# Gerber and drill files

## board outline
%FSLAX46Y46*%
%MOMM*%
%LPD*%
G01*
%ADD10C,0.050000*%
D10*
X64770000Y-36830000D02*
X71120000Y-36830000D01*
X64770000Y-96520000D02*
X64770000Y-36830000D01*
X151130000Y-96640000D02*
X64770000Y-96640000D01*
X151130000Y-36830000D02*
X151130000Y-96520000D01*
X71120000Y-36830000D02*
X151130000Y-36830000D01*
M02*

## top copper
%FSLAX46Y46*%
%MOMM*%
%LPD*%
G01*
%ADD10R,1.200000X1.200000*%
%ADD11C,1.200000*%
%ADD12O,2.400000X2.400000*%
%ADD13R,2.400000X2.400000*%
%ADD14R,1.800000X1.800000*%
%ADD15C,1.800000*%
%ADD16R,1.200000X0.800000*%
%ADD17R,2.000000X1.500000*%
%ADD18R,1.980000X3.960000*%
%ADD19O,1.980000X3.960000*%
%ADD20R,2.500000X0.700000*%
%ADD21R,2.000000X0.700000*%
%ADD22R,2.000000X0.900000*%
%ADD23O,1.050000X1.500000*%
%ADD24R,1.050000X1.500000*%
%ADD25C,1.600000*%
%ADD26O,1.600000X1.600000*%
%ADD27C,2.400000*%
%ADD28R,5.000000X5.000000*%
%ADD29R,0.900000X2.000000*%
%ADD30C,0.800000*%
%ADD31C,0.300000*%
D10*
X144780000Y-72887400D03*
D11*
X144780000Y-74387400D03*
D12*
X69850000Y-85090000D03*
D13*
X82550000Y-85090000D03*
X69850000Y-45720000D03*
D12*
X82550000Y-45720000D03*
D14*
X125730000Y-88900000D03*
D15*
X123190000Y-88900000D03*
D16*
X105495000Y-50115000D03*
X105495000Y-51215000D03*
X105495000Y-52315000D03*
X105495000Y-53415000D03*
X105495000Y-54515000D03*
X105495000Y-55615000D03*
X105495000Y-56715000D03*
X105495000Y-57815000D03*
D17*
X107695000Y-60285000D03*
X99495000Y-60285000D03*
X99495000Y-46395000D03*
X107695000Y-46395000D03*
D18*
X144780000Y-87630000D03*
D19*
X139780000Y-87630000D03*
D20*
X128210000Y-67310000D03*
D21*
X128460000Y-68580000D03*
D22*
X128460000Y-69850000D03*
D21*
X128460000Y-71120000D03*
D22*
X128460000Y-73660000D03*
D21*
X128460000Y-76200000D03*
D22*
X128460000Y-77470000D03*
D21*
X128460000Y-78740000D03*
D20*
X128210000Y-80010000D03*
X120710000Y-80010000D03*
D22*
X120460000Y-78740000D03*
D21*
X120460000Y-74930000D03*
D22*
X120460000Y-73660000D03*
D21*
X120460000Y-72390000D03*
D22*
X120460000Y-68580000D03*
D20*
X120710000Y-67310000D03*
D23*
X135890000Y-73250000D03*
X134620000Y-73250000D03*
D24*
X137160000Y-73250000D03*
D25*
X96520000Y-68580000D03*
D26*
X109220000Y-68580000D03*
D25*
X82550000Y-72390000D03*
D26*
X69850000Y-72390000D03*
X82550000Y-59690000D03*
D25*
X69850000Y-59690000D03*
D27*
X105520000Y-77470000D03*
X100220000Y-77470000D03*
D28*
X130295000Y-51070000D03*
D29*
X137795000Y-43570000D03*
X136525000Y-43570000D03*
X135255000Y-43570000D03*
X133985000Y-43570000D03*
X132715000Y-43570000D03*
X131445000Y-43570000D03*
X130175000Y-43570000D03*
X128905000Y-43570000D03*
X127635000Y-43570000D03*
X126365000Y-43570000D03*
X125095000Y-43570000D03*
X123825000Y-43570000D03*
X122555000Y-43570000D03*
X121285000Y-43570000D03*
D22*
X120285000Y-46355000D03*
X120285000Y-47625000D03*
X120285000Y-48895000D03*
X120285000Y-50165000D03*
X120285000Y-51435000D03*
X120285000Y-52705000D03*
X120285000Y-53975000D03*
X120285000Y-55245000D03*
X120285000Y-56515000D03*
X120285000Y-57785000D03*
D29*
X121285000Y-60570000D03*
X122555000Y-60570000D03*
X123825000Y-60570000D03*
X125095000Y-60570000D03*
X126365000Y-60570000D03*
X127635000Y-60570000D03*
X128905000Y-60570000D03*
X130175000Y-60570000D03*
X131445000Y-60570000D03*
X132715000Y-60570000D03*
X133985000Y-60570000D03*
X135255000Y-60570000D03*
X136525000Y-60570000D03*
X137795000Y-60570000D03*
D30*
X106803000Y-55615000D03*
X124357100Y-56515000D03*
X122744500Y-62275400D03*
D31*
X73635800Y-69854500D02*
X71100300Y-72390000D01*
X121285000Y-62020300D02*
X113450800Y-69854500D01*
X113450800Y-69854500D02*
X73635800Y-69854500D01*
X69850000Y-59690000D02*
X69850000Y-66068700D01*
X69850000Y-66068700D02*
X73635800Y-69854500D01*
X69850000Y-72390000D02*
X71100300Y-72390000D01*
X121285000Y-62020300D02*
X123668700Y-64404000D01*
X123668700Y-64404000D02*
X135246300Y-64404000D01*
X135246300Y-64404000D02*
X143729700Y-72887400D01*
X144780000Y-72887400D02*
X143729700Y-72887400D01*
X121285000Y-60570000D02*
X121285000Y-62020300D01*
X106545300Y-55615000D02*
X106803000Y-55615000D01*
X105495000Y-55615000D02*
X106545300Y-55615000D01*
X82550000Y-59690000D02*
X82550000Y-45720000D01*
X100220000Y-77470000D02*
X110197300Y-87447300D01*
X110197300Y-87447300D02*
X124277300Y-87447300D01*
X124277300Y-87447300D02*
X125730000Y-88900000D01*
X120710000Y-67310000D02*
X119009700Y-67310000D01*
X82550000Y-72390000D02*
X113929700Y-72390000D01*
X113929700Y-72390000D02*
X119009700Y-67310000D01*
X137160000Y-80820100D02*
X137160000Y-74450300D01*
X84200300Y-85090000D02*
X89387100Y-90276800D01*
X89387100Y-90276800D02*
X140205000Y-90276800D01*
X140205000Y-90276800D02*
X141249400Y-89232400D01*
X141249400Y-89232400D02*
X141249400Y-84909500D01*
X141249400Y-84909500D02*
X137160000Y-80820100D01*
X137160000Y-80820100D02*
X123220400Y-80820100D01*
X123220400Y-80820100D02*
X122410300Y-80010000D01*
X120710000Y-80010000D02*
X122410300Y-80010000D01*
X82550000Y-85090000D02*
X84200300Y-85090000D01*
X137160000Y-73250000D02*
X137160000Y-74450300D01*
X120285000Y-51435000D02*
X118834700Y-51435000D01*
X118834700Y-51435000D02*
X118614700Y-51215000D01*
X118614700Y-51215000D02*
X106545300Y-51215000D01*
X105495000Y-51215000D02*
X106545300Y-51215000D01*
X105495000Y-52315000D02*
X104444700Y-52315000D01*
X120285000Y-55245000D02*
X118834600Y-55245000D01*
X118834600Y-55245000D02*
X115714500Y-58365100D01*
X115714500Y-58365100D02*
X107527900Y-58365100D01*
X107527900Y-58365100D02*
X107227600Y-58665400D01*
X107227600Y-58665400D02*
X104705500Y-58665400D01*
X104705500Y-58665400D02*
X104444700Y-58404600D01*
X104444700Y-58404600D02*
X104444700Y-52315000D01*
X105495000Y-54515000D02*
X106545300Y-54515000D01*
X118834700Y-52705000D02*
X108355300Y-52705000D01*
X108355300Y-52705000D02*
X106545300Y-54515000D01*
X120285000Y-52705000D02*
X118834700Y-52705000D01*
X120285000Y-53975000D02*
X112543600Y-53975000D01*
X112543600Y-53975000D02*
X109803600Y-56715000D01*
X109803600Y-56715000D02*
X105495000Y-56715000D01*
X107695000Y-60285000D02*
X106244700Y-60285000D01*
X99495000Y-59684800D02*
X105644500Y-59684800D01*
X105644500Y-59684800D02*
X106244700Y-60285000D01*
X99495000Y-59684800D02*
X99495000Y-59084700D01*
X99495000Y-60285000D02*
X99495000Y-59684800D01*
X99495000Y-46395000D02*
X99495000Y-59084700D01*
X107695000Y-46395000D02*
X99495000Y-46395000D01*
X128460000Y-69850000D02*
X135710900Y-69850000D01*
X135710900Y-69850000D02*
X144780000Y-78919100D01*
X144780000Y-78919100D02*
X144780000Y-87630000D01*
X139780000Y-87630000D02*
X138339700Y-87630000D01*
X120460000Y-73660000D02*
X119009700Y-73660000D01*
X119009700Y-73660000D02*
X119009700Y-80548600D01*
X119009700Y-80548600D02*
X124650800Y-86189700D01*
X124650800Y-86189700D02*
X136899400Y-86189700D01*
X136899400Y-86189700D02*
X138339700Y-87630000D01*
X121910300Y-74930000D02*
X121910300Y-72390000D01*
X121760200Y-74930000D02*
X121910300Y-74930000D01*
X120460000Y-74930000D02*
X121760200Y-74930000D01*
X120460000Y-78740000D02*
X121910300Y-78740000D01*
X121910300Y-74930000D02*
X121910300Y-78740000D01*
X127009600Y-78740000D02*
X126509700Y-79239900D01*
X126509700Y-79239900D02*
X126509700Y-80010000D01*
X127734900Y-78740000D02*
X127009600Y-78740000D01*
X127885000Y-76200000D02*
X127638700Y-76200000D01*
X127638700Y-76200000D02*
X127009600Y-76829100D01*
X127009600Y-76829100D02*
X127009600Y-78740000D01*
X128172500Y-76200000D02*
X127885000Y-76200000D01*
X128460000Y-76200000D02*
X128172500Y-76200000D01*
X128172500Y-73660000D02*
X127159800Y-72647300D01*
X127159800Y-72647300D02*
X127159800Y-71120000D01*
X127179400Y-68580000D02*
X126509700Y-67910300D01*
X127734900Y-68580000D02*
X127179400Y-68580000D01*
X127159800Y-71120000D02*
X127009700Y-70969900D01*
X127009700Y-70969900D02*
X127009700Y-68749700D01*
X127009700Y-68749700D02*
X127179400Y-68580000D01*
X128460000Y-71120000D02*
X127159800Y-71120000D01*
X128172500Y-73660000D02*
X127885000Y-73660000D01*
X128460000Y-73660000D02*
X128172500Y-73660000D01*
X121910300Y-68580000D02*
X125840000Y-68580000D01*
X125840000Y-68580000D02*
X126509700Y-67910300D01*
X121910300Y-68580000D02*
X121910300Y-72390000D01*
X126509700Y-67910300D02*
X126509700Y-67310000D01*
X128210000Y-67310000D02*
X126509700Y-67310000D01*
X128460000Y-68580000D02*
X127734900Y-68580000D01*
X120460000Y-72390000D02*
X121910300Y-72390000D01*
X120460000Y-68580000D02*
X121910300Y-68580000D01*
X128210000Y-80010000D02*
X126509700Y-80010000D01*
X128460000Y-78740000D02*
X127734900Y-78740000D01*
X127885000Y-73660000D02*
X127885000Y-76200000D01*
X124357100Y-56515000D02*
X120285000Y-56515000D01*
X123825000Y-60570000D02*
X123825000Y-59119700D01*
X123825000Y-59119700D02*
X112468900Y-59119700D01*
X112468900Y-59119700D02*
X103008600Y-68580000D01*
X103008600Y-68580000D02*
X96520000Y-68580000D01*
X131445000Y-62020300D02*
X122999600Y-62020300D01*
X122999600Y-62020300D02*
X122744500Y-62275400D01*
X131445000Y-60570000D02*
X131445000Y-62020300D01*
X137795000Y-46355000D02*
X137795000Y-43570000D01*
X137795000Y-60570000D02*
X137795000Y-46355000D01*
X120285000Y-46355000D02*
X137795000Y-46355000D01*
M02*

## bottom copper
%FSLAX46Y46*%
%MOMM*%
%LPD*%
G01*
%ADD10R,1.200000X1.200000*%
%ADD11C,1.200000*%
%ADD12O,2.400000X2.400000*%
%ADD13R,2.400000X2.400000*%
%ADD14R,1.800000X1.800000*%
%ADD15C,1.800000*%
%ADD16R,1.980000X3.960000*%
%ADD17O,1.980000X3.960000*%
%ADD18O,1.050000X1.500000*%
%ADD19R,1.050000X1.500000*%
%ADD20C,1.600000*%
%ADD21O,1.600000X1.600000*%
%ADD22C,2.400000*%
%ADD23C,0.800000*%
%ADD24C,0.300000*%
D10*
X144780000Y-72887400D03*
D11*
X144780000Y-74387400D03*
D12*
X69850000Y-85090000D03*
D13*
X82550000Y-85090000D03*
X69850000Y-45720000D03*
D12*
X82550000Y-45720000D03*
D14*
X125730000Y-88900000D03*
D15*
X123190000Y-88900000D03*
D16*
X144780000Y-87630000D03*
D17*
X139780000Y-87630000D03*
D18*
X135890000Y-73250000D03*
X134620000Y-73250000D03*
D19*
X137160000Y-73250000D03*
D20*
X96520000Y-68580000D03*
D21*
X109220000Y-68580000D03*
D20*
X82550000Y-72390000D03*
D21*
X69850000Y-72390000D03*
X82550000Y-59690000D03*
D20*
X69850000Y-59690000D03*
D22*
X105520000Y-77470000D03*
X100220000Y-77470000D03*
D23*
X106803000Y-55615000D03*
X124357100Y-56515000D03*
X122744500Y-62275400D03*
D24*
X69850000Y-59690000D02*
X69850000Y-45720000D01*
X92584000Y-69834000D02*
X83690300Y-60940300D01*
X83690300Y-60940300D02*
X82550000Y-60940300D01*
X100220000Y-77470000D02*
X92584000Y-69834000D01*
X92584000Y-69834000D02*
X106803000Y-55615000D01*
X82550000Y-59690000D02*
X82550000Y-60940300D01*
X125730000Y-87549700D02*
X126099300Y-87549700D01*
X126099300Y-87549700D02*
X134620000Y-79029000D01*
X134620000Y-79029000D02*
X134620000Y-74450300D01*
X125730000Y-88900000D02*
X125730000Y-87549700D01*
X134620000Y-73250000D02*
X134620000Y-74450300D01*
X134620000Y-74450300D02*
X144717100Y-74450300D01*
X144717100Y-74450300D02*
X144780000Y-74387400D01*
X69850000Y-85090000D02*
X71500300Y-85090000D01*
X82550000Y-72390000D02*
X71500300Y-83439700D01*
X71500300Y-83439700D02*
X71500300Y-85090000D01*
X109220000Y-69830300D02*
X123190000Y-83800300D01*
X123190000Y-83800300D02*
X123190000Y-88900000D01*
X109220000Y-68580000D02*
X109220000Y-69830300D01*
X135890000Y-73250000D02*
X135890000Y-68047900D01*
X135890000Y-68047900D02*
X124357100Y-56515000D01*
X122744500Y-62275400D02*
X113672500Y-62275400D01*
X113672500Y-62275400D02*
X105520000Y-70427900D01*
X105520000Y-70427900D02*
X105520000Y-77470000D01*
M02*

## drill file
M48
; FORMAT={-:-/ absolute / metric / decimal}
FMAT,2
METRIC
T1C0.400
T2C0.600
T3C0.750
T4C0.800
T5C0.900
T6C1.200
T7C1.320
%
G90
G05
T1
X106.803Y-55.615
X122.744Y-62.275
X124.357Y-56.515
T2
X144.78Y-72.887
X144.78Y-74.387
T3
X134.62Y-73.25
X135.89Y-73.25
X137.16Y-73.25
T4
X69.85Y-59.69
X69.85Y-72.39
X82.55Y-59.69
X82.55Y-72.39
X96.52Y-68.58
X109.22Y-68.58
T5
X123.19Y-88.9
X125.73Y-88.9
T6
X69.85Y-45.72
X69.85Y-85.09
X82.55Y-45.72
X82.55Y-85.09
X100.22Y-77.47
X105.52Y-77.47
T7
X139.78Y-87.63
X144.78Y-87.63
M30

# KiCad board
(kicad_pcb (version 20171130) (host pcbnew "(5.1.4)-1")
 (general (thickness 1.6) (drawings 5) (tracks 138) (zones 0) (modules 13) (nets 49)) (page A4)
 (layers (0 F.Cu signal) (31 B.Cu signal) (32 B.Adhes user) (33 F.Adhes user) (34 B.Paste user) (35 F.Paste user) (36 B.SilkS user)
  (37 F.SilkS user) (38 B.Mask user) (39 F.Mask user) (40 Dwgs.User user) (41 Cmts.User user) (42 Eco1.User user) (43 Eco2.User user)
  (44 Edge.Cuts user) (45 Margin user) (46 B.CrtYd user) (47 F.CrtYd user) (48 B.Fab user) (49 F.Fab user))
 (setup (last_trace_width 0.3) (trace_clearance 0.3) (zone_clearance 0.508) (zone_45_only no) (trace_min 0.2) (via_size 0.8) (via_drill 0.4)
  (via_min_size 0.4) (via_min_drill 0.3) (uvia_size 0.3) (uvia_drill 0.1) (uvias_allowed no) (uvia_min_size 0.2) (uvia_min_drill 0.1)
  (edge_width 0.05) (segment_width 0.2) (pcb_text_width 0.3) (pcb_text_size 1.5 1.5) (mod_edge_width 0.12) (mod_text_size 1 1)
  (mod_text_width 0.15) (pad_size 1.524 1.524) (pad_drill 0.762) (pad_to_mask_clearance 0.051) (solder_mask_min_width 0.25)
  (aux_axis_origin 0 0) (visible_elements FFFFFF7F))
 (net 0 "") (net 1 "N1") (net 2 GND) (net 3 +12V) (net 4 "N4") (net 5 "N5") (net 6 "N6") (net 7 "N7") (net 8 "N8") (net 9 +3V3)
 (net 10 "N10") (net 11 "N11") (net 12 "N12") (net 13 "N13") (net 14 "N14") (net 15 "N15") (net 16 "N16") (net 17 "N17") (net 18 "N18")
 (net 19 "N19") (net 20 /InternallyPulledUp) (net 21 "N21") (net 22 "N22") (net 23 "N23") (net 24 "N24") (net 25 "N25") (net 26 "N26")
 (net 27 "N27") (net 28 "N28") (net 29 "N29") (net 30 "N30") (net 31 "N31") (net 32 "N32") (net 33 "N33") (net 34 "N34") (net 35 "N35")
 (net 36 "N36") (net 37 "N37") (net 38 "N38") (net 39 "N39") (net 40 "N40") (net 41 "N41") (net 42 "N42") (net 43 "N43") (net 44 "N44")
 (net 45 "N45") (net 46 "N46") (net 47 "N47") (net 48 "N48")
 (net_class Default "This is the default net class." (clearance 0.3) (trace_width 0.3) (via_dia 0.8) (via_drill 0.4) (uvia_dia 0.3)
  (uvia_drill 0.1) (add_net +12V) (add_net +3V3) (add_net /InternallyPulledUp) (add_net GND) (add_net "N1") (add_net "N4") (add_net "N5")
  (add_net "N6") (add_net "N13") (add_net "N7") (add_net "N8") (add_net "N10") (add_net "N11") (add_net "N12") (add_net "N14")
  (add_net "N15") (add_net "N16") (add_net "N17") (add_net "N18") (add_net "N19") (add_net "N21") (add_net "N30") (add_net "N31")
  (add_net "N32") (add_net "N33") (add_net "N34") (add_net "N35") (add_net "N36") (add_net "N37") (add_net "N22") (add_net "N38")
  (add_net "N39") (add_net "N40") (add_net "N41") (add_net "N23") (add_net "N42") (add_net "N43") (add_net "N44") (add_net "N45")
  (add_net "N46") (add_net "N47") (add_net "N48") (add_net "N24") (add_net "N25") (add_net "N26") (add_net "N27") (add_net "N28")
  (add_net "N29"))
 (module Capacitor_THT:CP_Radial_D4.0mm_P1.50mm (layer F.Cu) (at 144.78 72.8874 270)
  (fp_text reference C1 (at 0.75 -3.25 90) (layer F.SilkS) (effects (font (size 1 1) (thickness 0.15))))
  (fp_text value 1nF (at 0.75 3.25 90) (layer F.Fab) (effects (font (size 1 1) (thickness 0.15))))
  (pad 1 thru_hole rect (at 0 0 270) (size 1.2 1.2) (drill 0.6) (layers *.Cu *.Mask) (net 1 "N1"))
  (pad 2 thru_hole circle (at 1.5 0 270) (size 1.2 1.2) (drill 0.6) (layers *.Cu *.Mask) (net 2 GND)))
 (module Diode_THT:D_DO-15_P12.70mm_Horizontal (layer F.Cu) (at 82.55 85.09 180)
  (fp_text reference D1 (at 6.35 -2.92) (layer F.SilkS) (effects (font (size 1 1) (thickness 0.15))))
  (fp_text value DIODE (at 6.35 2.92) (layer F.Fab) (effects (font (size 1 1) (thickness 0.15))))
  (pad 2 thru_hole oval (at 12.7 0 180) (size 2.4 2.4) (drill 1.2) (layers *.Cu *.Mask) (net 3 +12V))
  (pad 1 thru_hole rect (at 0 0 180) (size 2.4 2.4) (drill 1.2) (layers *.Cu *.Mask) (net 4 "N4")))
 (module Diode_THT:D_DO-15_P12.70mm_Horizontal (layer F.Cu) (at 69.85 45.72)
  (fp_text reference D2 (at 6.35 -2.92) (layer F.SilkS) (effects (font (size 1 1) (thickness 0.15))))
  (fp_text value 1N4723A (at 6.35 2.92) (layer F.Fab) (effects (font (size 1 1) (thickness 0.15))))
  (pad 1 thru_hole rect (at 0 0) (size 2.4 2.4) (drill 1.2) (layers *.Cu *.Mask) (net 1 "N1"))
  (pad 2 thru_hole oval (at 12.7 0) (size 2.4 2.4) (drill 1.2) (layers *.Cu *.Mask) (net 2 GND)))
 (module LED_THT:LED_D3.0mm (layer F.Cu) (at 125.73 88.9 180)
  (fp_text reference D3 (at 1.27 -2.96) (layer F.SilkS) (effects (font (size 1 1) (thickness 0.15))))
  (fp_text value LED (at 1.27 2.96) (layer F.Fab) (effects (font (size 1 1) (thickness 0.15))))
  (pad 1 thru_hole rect (at 0 0 180) (size 1.8 1.8) (drill 0.9) (layers *.Cu *.Mask) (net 2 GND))
  (pad 2 thru_hole circle (at 2.54 0 180) (size 1.8 1.8) (drill 0.9) (layers *.Cu *.Mask) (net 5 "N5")))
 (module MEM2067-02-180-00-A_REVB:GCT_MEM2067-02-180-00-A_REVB (layer F.Cu) (at 102.87 53.34 90)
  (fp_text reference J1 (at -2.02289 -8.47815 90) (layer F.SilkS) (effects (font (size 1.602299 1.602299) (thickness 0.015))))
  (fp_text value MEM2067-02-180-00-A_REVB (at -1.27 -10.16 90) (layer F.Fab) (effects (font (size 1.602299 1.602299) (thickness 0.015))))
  (pad 1 smd rect (at 3.225 2.625 90) (size 0.8 1.2) (layers F.Cu F.Paste F.Mask) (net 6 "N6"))
  (pad 2 smd rect (at 2.125 2.625 90) (size 0.8 1.2) (layers F.Cu F.Paste F.Mask) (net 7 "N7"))
  (pad 3 smd rect (at 1.025 2.625 90) (size 0.8 1.2) (layers F.Cu F.Paste F.Mask) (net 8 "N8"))
  (pad 4 smd rect (at -0.075 2.625 90) (size 0.8 1.2) (layers F.Cu F.Paste F.Mask) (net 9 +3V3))
  (pad 5 smd rect (at -1.175 2.625 90) (size 0.8 1.2) (layers F.Cu F.Paste F.Mask) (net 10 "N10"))
  (pad 6 smd rect (at -2.275 2.625 90) (size 0.8 1.2) (layers F.Cu F.Paste F.Mask) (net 2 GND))
  (pad 7 smd rect (at -3.375 2.625 90) (size 0.8 1.2) (layers F.Cu F.Paste F.Mask) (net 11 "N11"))
  (pad 8 smd rect (at -4.475 2.625 90) (size 0.8 1.2) (layers F.Cu F.Paste F.Mask) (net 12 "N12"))
  (pad 9 smd rect (at -6.945 4.825 90) (size 1.5 2) (layers F.Cu F.Paste F.Mask) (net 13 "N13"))
  (pad 10 smd rect (at -6.945 -3.375 90) (size 1.5 2) (layers F.Cu F.Paste F.Mask) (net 13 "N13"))
  (pad 11 smd rect (at 6.945 -3.375 90) (size 1.5 2) (layers F.Cu F.Paste F.Mask) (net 13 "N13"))
  (pad 12 smd rect (at 6.945 4.825 90) (size 1.5 2) (layers F.Cu F.Paste F.Mask) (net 13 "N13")))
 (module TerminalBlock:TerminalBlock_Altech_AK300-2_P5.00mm (layer F.Cu) (at 144.78 87.63 180)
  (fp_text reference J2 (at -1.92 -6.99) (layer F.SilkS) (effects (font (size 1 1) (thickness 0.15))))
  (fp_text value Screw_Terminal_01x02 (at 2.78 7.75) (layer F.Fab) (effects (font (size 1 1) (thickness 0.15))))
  (pad 1 thru_hole rect (at 0 0 180) (size 1.98 3.96) (drill 1.32) (layers *.Cu *.Mask) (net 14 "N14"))
  (pad 2 thru_hole oval (at 5 0 180) (size 1.98 3.96) (drill 1.32) (layers *.Cu *.Mask) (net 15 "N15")))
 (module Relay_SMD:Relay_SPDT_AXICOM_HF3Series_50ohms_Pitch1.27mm (layer F.Cu) (at 124.46 73.66)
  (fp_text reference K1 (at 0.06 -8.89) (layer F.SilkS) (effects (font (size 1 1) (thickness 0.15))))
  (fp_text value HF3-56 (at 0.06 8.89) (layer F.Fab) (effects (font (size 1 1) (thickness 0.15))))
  (pad 22 smd rect (at 3.75 -6.35) (size 2.5 0.7) (layers F.Cu F.Paste F.Mask) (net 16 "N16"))
  (pad 21 smd rect (at 4 -5.08) (size 2 0.7) (layers F.Cu F.Paste F.Mask) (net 16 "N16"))
  (pad 20 smd rect (at 4 -3.81) (size 2 0.9) (layers F.Cu F.Paste F.Mask) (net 14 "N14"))
  (pad 19 smd rect (at 4 -2.54) (size 2 0.7) (layers F.Cu F.Paste F.Mask) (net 16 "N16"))
  (pad 17 smd rect (at 4 0) (size 2 0.9) (layers F.Cu F.Paste F.Mask) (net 16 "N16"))
  (pad 15 smd rect (at 4 2.54) (size 2 0.7) (layers F.Cu F.Paste F.Mask) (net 16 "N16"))
  (pad 14 smd rect (at 4 3.81) (size 2 0.9) (layers F.Cu F.Paste F.Mask) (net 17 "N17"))
  (pad 13 smd rect (at 4 5.08) (size 2 0.7) (layers F.Cu F.Paste F.Mask) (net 16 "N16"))
  (pad 12 smd rect (at 3.75 6.35) (size 2.5 0.7) (layers F.Cu F.Paste F.Mask) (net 16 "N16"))
  (pad 11 smd rect (at -3.75 6.35) (size 2.5 0.7) (layers F.Cu F.Paste F.Mask) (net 4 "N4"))
  (pad 10 smd rect (at -4 5.08) (size 2 0.9) (layers F.Cu F.Paste F.Mask) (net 16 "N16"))
  (pad 7 smd rect (at -4 1.27) (size 2 0.7) (layers F.Cu F.Paste F.Mask) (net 16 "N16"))
  (pad 6 smd rect (at -4 0) (size 2 0.9) (layers F.Cu F.Paste F.Mask) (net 15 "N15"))
  (pad 5 smd rect (at -4 -1.27) (size 2 0.7) (layers F.Cu F.Paste F.Mask) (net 16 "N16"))
  (pad 2 smd rect (at -4 -5.08) (size 2 0.9) (layers F.Cu F.Paste F.Mask) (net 16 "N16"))
  (pad 1 smd rect (at -3.75 -6.35) (size 2.5 0.7) (layers F.Cu F.Paste F.Mask) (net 3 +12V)))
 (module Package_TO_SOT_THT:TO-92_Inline (layer F.Cu) (at 137.16 73.25 180)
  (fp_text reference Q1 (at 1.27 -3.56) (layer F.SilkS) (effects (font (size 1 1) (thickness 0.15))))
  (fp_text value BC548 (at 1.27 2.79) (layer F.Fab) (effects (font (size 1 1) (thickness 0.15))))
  (pad 2 thru_hole oval (at 1.27 0 180) (size 1.05 1.5) (drill 0.75) (layers *.Cu *.Mask) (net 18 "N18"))
  (pad 3 thru_hole oval (at 2.54 0 180) (size 1.05 1.5) (drill 0.75) (layers *.Cu *.Mask) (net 2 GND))
  (pad 1 thru_hole rect (at 0 0 180) (size 1.05 1.5) (drill 0.75) (layers *.Cu *.Mask) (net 4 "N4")))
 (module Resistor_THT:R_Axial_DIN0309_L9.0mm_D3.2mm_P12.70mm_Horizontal (layer F.Cu) (at 96.52 68.58)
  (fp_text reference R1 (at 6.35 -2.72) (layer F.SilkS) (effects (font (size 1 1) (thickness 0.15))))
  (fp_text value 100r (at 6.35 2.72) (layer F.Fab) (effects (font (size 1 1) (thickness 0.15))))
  (pad 1 thru_hole circle (at 0 0) (size 1.6 1.6) (drill 0.8) (layers *.Cu *.Mask) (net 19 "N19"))
  (pad 2 thru_hole oval (at 12.7 0) (size 1.6 1.6) (drill 0.8) (layers *.Cu *.Mask) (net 5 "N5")))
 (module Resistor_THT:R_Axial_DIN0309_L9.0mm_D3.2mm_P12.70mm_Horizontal (layer F.Cu) (at 82.55 72.39 180)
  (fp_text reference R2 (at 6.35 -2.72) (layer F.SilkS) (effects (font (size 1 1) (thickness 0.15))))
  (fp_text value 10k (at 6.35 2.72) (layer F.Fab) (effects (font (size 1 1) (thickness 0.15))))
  (pad 1 thru_hole circle (at 0 0 180) (size 1.6 1.6) (drill 0.8) (layers *.Cu *.Mask) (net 3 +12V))
  (pad 2 thru_hole oval (at 12.7 0 180) (size 1.6 1.6) (drill 0.8) (layers *.Cu *.Mask) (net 1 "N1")))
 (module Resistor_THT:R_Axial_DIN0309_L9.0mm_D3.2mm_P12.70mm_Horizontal (layer F.Cu) (at 69.85 59.69)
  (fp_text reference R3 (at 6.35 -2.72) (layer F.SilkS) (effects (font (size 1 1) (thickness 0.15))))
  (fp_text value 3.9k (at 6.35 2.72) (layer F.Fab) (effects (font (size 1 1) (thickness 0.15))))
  (pad 2 thru_hole oval (at 12.7 0) (size 1.6 1.6) (drill 0.8) (layers *.Cu *.Mask) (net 2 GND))
  (pad 1 thru_hole circle (at 0 0) (size 1.6 1.6) (drill 0.8) (layers *.Cu *.Mask) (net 1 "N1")))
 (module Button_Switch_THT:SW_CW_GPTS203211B (layer F.Cu) (at 105.52 77.47 270)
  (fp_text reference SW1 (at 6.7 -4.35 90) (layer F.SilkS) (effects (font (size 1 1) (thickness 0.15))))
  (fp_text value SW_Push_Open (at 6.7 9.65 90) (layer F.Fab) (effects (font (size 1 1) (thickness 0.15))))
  (pad 1 thru_hole circle (at 0 0 270) (size 2.4 2.4) (drill 1.2) (layers *.Cu *.Mask) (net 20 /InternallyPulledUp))
  (pad 2 thru_hole circle (at 0 5.3 270) (size 2.4 2.4) (drill 1.2) (layers *.Cu *.Mask) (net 2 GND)))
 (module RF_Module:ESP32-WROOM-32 (layer F.Cu) (at 129.54 52.07 270)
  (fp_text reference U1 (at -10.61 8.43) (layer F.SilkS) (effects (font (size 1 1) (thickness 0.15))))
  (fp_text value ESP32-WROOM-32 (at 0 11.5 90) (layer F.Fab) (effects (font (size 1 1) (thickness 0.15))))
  (pad 39 smd rect (at -1 -0.755 270) (size 5 5) (layers F.Cu F.Paste F.Mask))
  (pad 1 smd rect (at -8.5 -8.255 270) (size 2 0.9) (layers F.Cu F.Paste F.Mask) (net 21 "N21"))
  (pad 2 smd rect (at -8.5 -6.985 270) (size 2 0.9) (layers F.Cu F.Paste F.Mask) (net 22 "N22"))
  (pad 3 smd rect (at -8.5 -5.715 270) (size 2 0.9) (layers F.Cu F.Paste F.Mask) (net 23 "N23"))
  (pad 4 smd rect (at -8.5 -4.445 270) (size 2 0.9) (layers F.Cu F.Paste F.Mask) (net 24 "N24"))
  (pad 5 smd rect (at -8.5 -3.175 270) (size 2 0.9) (layers F.Cu F.Paste F.Mask) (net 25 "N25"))
  (pad 6 smd rect (at -8.5 -1.905 270) (size 2 0.9) (layers F.Cu F.Paste F.Mask) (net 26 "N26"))
  (pad 7 smd rect (at -8.5 -0.635 270) (size 2 0.9) (layers F.Cu F.Paste F.Mask) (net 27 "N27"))
  (pad 8 smd rect (at -8.5 0.635 270) (size 2 0.9) (layers F.Cu F.Paste F.Mask) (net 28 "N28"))
  (pad 9 smd rect (at -8.5 1.905 270) (size 2 0.9) (layers F.Cu F.Paste F.Mask) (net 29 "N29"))
  (pad 10 smd rect (at -8.5 3.175 270) (size 2 0.9) (layers F.Cu F.Paste F.Mask) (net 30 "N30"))
  (pad 11 smd rect (at -8.5 4.445 270) (size 2 0.9) (layers F.Cu F.Paste F.Mask) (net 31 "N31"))
  (pad 12 smd rect (at -8.5 5.715 270) (size 2 0.9) (layers F.Cu F.Paste F.Mask) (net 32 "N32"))
  (pad 13 smd rect (at -8.5 6.985 270) (size 2 0.9) (layers F.Cu F.Paste F.Mask) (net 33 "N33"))
  (pad 14 smd rect (at -8.5 8.255 270) (size 2 0.9) (layers F.Cu F.Paste F.Mask) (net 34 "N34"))
  (pad 15 smd rect (at -5.715 9.255) (size 2 0.9) (layers F.Cu F.Paste F.Mask) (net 21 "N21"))
  (pad 16 smd rect (at -4.445 9.255) (size 2 0.9) (layers F.Cu F.Paste F.Mask) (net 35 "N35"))
  (pad 17 smd rect (at -3.175 9.255) (size 2 0.9) (layers F.Cu F.Paste F.Mask) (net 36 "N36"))
  (pad 18 smd rect (at -1.905 9.255) (size 2 0.9) (layers F.Cu F.Paste F.Mask) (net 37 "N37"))
  (pad 19 smd rect (at -0.635 9.255) (size 2 0.9) (layers F.Cu F.Paste F.Mask) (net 7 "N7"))
  (pad 20 smd rect (at 0.635 9.255) (size 2 0.9) (layers F.Cu F.Paste F.Mask) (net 10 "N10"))
  (pad 21 smd rect (at 1.905 9.255) (size 2 0.9) (layers F.Cu F.Paste F.Mask) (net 11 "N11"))
  (pad 22 smd rect (at 3.175 9.255) (size 2 0.9) (layers F.Cu F.Paste F.Mask) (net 8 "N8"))
  (pad 23 smd rect (at 4.445 9.255) (size 2 0.9) (layers F.Cu F.Paste F.Mask) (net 18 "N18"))
  (pad 24 smd rect (at 5.715 9.255) (size 2 0.9) (layers F.Cu F.Paste F.Mask) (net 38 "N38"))
  (pad 25 smd rect (at 8.5 8.255 270) (size 2 0.9) (layers F.Cu F.Paste F.Mask) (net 1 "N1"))
  (pad 26 smd rect (at 8.5 6.985 270) (size 2 0.9) (layers F.Cu F.Paste F.Mask) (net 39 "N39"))
  (pad 27 smd rect (at 8.5 5.715 270) (size 2 0.9) (layers F.Cu F.Paste F.Mask) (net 19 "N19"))
  (pad 28 smd rect (at 8.5 4.445 270) (size 2 0.9) (layers F.Cu F.Paste F.Mask) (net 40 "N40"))
  (pad 29 smd rect (at 8.5 3.175 270) (size 2 0.9) (layers F.Cu F.Paste F.Mask) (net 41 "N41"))
  (pad 30 smd rect (at 8.5 1.905 270) (size 2 0.9) (layers F.Cu F.Paste F.Mask) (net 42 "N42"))
  (pad 31 smd rect (at 8.5 0.635 270) (size 2 0.9) (layers F.Cu F.Paste F.Mask) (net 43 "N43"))
  (pad 32 smd rect (at 8.5 -0.635 270) (size 2 0.9) (layers F.Cu F.Paste F.Mask) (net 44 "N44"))
  (pad 33 smd rect (at 8.5 -1.905 270) (size 2 0.9) (layers F.Cu F.Paste F.Mask) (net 20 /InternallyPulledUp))
  (pad 34 smd rect (at 8.5 -3.175 270) (size 2 0.9) (layers F.Cu F.Paste F.Mask) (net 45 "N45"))
  (pad 35 smd rect (at 8.5 -4.445 270) (size 2 0.9) (layers F.Cu F.Paste F.Mask) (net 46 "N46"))
  (pad 36 smd rect (at 8.5 -5.715 270) (size 2 0.9) (layers F.Cu F.Paste F.Mask) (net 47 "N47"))
  (pad 37 smd rect (at 8.5 -6.985 270) (size 2 0.9) (layers F.Cu F.Paste F.Mask) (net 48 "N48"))
  (pad 38 smd rect (at 8.5 -8.255 270) (size 2 0.9) (layers F.Cu F.Paste F.Mask) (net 21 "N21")))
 (gr_line (start 64.77 36.83) (end 71.12 36.83) (layer Edge.Cuts) (width 0.05))
 (gr_line (start 64.77 96.52) (end 64.77 36.83) (layer Edge.Cuts) (width 0.05))
 (gr_line (start 151.13 96.64) (end 64.77 96.64) (layer Edge.Cuts) (width 0.05))
 (gr_line (start 151.13 36.83) (end 151.13 96.52) (layer Edge.Cuts) (width 0.05))
 (gr_line (start 71.12 36.83) (end 151.13 36.83) (layer Edge.Cuts) (width 0.05))
 (segment (start 73.6358 69.8545) (end 71.1003 72.39) (width 0.3) (layer F.Cu) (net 1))
 (segment (start 121.285 62.0203) (end 113.4508 69.8545) (width 0.3) (layer F.Cu) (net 1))
 (segment (start 113.4508 69.8545) (end 73.6358 69.8545) (width 0.3) (layer F.Cu) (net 1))
 (segment (start 69.85 59.69) (end 69.85 66.0687) (width 0.3) (layer F.Cu) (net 1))
 (segment (start 69.85 66.0687) (end 73.6358 69.8545) (width 0.3) (layer F.Cu) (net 1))
 (segment (start 69.85 72.39) (end 71.1003 72.39) (width 0.3) (layer F.Cu) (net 1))
 (segment (start 121.285 62.0203) (end 123.6687 64.404) (width 0.3) (layer F.Cu) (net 1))
 (segment (start 123.6687 64.404) (end 135.2463 64.404) (width 0.3) (layer F.Cu) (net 1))
 (segment (start 135.2463 64.404) (end 143.7297 72.8874) (width 0.3) (layer F.Cu) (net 1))
 (segment (start 144.78 72.8874) (end 143.7297 72.8874) (width 0.3) (layer F.Cu) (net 1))
 (segment (start 121.285 60.57) (end 121.285 62.0203) (width 0.3) (layer F.Cu) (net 1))
 (segment (start 69.85 59.69) (end 69.85 45.72) (width 0.3) (layer B.Cu) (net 1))
 (segment (start 92.584 69.834) (end 83.6903 60.9403) (width 0.3) (layer B.Cu) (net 2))
 (segment (start 83.6903 60.9403) (end 82.55 60.9403) (width 0.3) (layer B.Cu) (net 2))
 (segment (start 100.22 77.47) (end 92.584 69.834) (width 0.3) (layer B.Cu) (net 2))
 (segment (start 92.584 69.834) (end 106.803 55.615) (width 0.3) (layer B.Cu) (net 2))
 (segment (start 106.5453 55.615) (end 106.803 55.615) (width 0.3) (layer F.Cu) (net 2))
 (segment (start 105.495 55.615) (end 106.5453 55.615) (width 0.3) (layer F.Cu) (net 2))
 (segment (start 82.55 59.69) (end 82.55 45.72) (width 0.3) (layer F.Cu) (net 2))
 (segment (start 82.55 59.69) (end 82.55 60.9403) (width 0.3) (layer B.Cu) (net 2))
 (segment (start 100.22 77.47) (end 110.1973 87.4473) (width 0.3) (layer F.Cu) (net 2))
 (segment (start 110.1973 87.4473) (end 124.2773 87.4473) (width 0.3) (layer F.Cu) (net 2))
 (segment (start 124.2773 87.4473) (end 125.73 88.9) (width 0.3) (layer F.Cu) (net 2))
 (segment (start 125.73 87.5497) (end 126.0993 87.5497) (width 0.3) (layer B.Cu) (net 2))
 (segment (start 126.0993 87.5497) (end 134.62 79.029) (width 0.3) (layer B.Cu) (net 2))
 (segment (start 134.62 79.029) (end 134.62 74.4503) (width 0.3) (layer B.Cu) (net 2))
 (segment (start 125.73 88.9) (end 125.73 87.5497) (width 0.3) (layer B.Cu) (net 2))
 (segment (start 134.62 73.25) (end 134.62 74.4503) (width 0.3) (layer B.Cu) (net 2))
 (segment (start 134.62 74.4503) (end 144.7171 74.4503) (width 0.3) (layer B.Cu) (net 2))
 (segment (start 144.7171 74.4503) (end 144.78 74.3874) (width 0.3) (layer B.Cu) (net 2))
 (via (at 106.803 55.615) (size 0.8) (layers F.Cu B.Cu) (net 2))
 (segment (start 120.71 67.31) (end 119.0097 67.31) (width 0.3) (layer F.Cu) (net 3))
 (segment (start 82.55 72.39) (end 113.9297 72.39) (width 0.3) (layer F.Cu) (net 3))
 (segment (start 113.9297 72.39) (end 119.0097 67.31) (width 0.3) (layer F.Cu) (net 3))
 (segment (start 69.85 85.09) (end 71.5003 85.09) (width 0.3) (layer B.Cu) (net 3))
 (segment (start 82.55 72.39) (end 71.5003 83.4397) (width 0.3) (layer B.Cu) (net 3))
 (segment (start 71.5003 83.4397) (end 71.5003 85.09) (width 0.3) (layer B.Cu) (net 3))
 (segment (start 137.16 80.8201) (end 137.16 74.4503) (width 0.3) (layer F.Cu) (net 4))
 (segment (start 84.2003 85.09) (end 89.3871 90.2768) (width 0.3) (layer F.Cu) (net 4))
 (segment (start 89.3871 90.2768) (end 140.205 90.2768) (width 0.3) (layer F.Cu) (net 4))
 (segment (start 140.205 90.2768) (end 141.2494 89.2324) (width 0.3) (layer F.Cu) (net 4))
 (segment (start 141.2494 89.2324) (end 141.2494 84.9095) (width 0.3) (layer F.Cu) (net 4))
 (segment (start 141.2494 84.9095) (end 137.16 80.8201) (width 0.3) (layer F.Cu) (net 4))
 (segment (start 137.16 80.8201) (end 123.2204 80.8201) (width 0.3) (layer F.Cu) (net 4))
 (segment (start 123.2204 80.8201) (end 122.4103 80.01) (width 0.3) (layer F.Cu) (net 4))
 (segment (start 120.71 80.01) (end 122.4103 80.01) (width 0.3) (layer F.Cu) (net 4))
 (segment (start 82.55 85.09) (end 84.2003 85.09) (width 0.3) (layer F.Cu) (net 4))
 (segment (start 137.16 73.25) (end 137.16 74.4503) (width 0.3) (layer F.Cu) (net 4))
 (segment (start 109.22 69.8303) (end 123.19 83.8003) (width 0.3) (layer B.Cu) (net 5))
 (segment (start 123.19 83.8003) (end 123.19 88.9) (width 0.3) (layer B.Cu) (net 5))
 (segment (start 109.22 68.58) (end 109.22 69.8303) (width 0.3) (layer B.Cu) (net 5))
 (segment (start 120.285 51.435) (end 118.8347 51.435) (width 0.3) (layer F.Cu) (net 7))
 (segment (start 118.8347 51.435) (end 118.6147 51.215) (width 0.3) (layer F.Cu) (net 7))
 (segment (start 118.6147 51.215) (end 106.5453 51.215) (width 0.3) (layer F.Cu) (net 7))
 (segment (start 105.495 51.215) (end 106.5453 51.215) (width 0.3) (layer F.Cu) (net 7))
 (segment (start 105.495 52.315) (end 104.4447 52.315) (width 0.3) (layer F.Cu) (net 8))
 (segment (start 120.285 55.245) (end 118.8346 55.245) (width 0.3) (layer F.Cu) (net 8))
 (segment (start 118.8346 55.245) (end 115.7145 58.3651) (width 0.3) (layer F.Cu) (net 8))
 (segment (start 115.7145 58.3651) (end 107.5279 58.3651) (width 0.3) (layer F.Cu) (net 8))
 (segment (start 107.5279 58.3651) (end 107.2276 58.6654) (width 0.3) (layer F.Cu) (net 8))
 (segment (start 107.2276 58.6654) (end 104.7055 58.6654) (width 0.3) (layer F.Cu) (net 8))
 (segment (start 104.7055 58.6654) (end 104.4447 58.4046) (width 0.3) (layer F.Cu) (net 8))
 (segment (start 104.4447 58.4046) (end 104.4447 52.315) (width 0.3) (layer F.Cu) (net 8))
 (segment (start 105.495 54.515) (end 106.5453 54.515) (width 0.3) (layer F.Cu) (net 10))
 (segment (start 118.8347 52.705) (end 108.3553 52.705) (width 0.3) (layer F.Cu) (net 10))
 (segment (start 108.3553 52.705) (end 106.5453 54.515) (width 0.3) (layer F.Cu) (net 10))
 (segment (start 120.285 52.705) (end 118.8347 52.705) (width 0.3) (layer F.Cu) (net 10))
 (segment (start 120.285 53.975) (end 112.5436 53.975) (width 0.3) (layer F.Cu) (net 11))
 (segment (start 112.5436 53.975) (end 109.8036 56.715) (width 0.3) (layer F.Cu) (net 11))
 (segment (start 109.8036 56.715) (end 105.495 56.715) (width 0.3) (layer F.Cu) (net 11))
 (segment (start 107.695 60.285) (end 106.2447 60.285) (width 0.3) (layer F.Cu) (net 13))
 (segment (start 99.495 59.6848) (end 105.6445 59.6848) (width 0.3) (layer F.Cu) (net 13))
 (segment (start 105.6445 59.6848) (end 106.2447 60.285) (width 0.3) (layer F.Cu) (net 13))
 (segment (start 99.495 59.6848) (end 99.495 59.0847) (width 0.3) (layer F.Cu) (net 13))
 (segment (start 99.495 60.285) (end 99.495 59.6848) (width 0.3) (layer F.Cu) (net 13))
 (segment (start 99.495 46.395) (end 99.495 59.0847) (width 0.3) (layer F.Cu) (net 13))
 (segment (start 107.695 46.395) (end 99.495 46.395) (width 0.3) (layer F.Cu) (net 13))
 (segment (start 128.46 69.85) (end 135.7109 69.85) (width 0.3) (layer F.Cu) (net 14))
 (segment (start 135.7109 69.85) (end 144.78 78.9191) (width 0.3) (layer F.Cu) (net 14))
 (segment (start 144.78 78.9191) (end 144.78 87.63) (width 0.3) (layer F.Cu) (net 14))
 (segment (start 139.78 87.63) (end 138.3397 87.63) (width 0.3) (layer F.Cu) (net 15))
 (segment (start 120.46 73.66) (end 119.0097 73.66) (width 0.3) (layer F.Cu) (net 15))
 (segment (start 119.0097 73.66) (end 119.0097 80.5486) (width 0.3) (layer F.Cu) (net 15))
 (segment (start 119.0097 80.5486) (end 124.6508 86.1897) (width 0.3) (layer F.Cu) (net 15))
 (segment (start 124.6508 86.1897) (end 136.8994 86.1897) (width 0.3) (layer F.Cu) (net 15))
 (segment (start 136.8994 86.1897) (end 138.3397 87.63) (width 0.3) (layer F.Cu) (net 15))
 (segment (start 121.9103 74.93) (end 121.9103 72.39) (width 0.3) (layer F.Cu) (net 16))
 (segment (start 121.7602 74.93) (end 121.9103 74.93) (width 0.3) (layer F.Cu) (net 16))
 (segment (start 120.46 74.93) (end 121.7602 74.93) (width 0.3) (layer F.Cu) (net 16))
 (segment (start 120.46 78.74) (end 121.9103 78.74) (width 0.3) (layer F.Cu) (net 16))
 (segment (start 121.9103 74.93) (end 121.9103 78.74) (width 0.3) (layer F.Cu) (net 16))
 (segment (start 127.0096 78.74) (end 126.5097 79.2399) (width 0.3) (layer F.Cu) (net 16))
 (segment (start 126.5097 79.2399) (end 126.5097 80.01) (width 0.3) (layer F.Cu) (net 16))
 (segment (start 127.7349 78.74) (end 127.0096 78.74) (width 0.3) (layer F.Cu) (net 16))
 (segment (start 127.885 76.2) (end 127.6387 76.2) (width 0.3) (layer F.Cu) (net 16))
 (segment (start 127.6387 76.2) (end 127.0096 76.8291) (width 0.3) (layer F.Cu) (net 16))
 (segment (start 127.0096 76.8291) (end 127.0096 78.74) (width 0.3) (layer F.Cu) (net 16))
 (segment (start 128.1725 76.2) (end 127.885 76.2) (width 0.3) (layer F.Cu) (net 16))
 (segment (start 128.46 76.2) (end 128.1725 76.2) (width 0.3) (layer F.Cu) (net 16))
 (segment (start 128.1725 73.66) (end 127.1598 72.6473) (width 0.3) (layer F.Cu) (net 16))
 (segment (start 127.1598 72.6473) (end 127.1598 71.12) (width 0.3) (layer F.Cu) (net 16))
 (segment (start 127.1794 68.58) (end 126.5097 67.9103) (width 0.3) (layer F.Cu) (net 16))
 (segment (start 127.7349 68.58) (end 127.1794 68.58) (width 0.3) (layer F.Cu) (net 16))
 (segment (start 127.1598 71.12) (end 127.0097 70.9699) (width 0.3) (layer F.Cu) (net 16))
 (segment (start 127.0097 70.9699) (end 127.0097 68.7497) (width 0.3) (layer F.Cu) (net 16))
 (segment (start 127.0097 68.7497) (end 127.1794 68.58) (width 0.3) (layer F.Cu) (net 16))
 (segment (start 128.46 71.12) (end 127.1598 71.12) (width 0.3) (layer F.Cu) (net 16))
 (segment (start 128.1725 73.66) (end 127.885 73.66) (width 0.3) (layer F.Cu) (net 16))
 (segment (start 128.46 73.66) (end 128.1725 73.66) (width 0.3) (layer F.Cu) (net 16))
 (segment (start 121.9103 68.58) (end 125.84 68.58) (width 0.3) (layer F.Cu) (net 16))
 (segment (start 125.84 68.58) (end 126.5097 67.9103) (width 0.3) (layer F.Cu) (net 16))
 (segment (start 121.9103 68.58) (end 121.9103 72.39) (width 0.3) (layer F.Cu) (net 16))
 (segment (start 126.5097 67.9103) (end 126.5097 67.31) (width 0.3) (layer F.Cu) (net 16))
 (segment (start 128.21 67.31) (end 126.5097 67.31) (width 0.3) (layer F.Cu) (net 16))
 (segment (start 128.46 68.58) (end 127.7349 68.58) (width 0.3) (layer F.Cu) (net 16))
 (segment (start 120.46 72.39) (end 121.9103 72.39) (width 0.3) (layer F.Cu) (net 16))
 (segment (start 120.46 68.58) (end 121.9103 68.58) (width 0.3) (layer F.Cu) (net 16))
 (segment (start 128.21 80.01) (end 126.5097 80.01) (width 0.3) (layer F.Cu) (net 16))
 (segment (start 128.46 78.74) (end 127.7349 78.74) (width 0.3) (layer F.Cu) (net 16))
 (segment (start 127.885 73.66) (end 127.885 76.2) (width 0.3) (layer F.Cu) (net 16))
 (segment (start 135.89 73.25) (end 135.89 68.0479) (width 0.3) (layer B.Cu) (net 18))
 (segment (start 135.89 68.0479) (end 124.3571 56.515) (width 0.3) (layer B.Cu) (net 18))
 (segment (start 124.3571 56.515) (end 120.285 56.515) (width 0.3) (layer F.Cu) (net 18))
 (via (at 124.3571 56.515) (size 0.8) (layers F.Cu B.Cu) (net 18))
 (segment (start 123.825 60.57) (end 123.825 59.1197) (width 0.3) (layer F.Cu) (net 19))
 (segment (start 123.825 59.1197) (end 112.4689 59.1197) (width 0.3) (layer F.Cu) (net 19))
 (segment (start 112.4689 59.1197) (end 103.0086 68.58) (width 0.3) (layer F.Cu) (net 19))
 (segment (start 103.0086 68.58) (end 96.52 68.58) (width 0.3) (layer F.Cu) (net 19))
 (segment (start 131.445 62.0203) (end 122.9996 62.0203) (width 0.3) (layer F.Cu) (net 20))
 (segment (start 122.9996 62.0203) (end 122.7445 62.2754) (width 0.3) (layer F.Cu) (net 20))
 (segment (start 122.7445 62.2754) (end 113.6725 62.2754) (width 0.3) (layer B.Cu) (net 20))
 (segment (start 113.6725 62.2754) (end 105.52 70.4279) (width 0.3) (layer B.Cu) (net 20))
 (segment (start 105.52 70.4279) (end 105.52 77.47) (width 0.3) (layer B.Cu) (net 20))
 (segment (start 131.445 60.57) (end 131.445 62.0203) (width 0.3) (layer F.Cu) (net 20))
 (via (at 122.7445 62.2754) (size 0.8) (layers F.Cu B.Cu) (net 20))
 (segment (start 137.795 46.355) (end 137.795 43.57) (width 0.3) (layer F.Cu) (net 21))
 (segment (start 137.795 60.57) (end 137.795 46.355) (width 0.3) (layer F.Cu) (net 21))
 (segment (start 120.285 46.355) (end 137.795 46.355) (width 0.3) (layer F.Cu) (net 21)))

